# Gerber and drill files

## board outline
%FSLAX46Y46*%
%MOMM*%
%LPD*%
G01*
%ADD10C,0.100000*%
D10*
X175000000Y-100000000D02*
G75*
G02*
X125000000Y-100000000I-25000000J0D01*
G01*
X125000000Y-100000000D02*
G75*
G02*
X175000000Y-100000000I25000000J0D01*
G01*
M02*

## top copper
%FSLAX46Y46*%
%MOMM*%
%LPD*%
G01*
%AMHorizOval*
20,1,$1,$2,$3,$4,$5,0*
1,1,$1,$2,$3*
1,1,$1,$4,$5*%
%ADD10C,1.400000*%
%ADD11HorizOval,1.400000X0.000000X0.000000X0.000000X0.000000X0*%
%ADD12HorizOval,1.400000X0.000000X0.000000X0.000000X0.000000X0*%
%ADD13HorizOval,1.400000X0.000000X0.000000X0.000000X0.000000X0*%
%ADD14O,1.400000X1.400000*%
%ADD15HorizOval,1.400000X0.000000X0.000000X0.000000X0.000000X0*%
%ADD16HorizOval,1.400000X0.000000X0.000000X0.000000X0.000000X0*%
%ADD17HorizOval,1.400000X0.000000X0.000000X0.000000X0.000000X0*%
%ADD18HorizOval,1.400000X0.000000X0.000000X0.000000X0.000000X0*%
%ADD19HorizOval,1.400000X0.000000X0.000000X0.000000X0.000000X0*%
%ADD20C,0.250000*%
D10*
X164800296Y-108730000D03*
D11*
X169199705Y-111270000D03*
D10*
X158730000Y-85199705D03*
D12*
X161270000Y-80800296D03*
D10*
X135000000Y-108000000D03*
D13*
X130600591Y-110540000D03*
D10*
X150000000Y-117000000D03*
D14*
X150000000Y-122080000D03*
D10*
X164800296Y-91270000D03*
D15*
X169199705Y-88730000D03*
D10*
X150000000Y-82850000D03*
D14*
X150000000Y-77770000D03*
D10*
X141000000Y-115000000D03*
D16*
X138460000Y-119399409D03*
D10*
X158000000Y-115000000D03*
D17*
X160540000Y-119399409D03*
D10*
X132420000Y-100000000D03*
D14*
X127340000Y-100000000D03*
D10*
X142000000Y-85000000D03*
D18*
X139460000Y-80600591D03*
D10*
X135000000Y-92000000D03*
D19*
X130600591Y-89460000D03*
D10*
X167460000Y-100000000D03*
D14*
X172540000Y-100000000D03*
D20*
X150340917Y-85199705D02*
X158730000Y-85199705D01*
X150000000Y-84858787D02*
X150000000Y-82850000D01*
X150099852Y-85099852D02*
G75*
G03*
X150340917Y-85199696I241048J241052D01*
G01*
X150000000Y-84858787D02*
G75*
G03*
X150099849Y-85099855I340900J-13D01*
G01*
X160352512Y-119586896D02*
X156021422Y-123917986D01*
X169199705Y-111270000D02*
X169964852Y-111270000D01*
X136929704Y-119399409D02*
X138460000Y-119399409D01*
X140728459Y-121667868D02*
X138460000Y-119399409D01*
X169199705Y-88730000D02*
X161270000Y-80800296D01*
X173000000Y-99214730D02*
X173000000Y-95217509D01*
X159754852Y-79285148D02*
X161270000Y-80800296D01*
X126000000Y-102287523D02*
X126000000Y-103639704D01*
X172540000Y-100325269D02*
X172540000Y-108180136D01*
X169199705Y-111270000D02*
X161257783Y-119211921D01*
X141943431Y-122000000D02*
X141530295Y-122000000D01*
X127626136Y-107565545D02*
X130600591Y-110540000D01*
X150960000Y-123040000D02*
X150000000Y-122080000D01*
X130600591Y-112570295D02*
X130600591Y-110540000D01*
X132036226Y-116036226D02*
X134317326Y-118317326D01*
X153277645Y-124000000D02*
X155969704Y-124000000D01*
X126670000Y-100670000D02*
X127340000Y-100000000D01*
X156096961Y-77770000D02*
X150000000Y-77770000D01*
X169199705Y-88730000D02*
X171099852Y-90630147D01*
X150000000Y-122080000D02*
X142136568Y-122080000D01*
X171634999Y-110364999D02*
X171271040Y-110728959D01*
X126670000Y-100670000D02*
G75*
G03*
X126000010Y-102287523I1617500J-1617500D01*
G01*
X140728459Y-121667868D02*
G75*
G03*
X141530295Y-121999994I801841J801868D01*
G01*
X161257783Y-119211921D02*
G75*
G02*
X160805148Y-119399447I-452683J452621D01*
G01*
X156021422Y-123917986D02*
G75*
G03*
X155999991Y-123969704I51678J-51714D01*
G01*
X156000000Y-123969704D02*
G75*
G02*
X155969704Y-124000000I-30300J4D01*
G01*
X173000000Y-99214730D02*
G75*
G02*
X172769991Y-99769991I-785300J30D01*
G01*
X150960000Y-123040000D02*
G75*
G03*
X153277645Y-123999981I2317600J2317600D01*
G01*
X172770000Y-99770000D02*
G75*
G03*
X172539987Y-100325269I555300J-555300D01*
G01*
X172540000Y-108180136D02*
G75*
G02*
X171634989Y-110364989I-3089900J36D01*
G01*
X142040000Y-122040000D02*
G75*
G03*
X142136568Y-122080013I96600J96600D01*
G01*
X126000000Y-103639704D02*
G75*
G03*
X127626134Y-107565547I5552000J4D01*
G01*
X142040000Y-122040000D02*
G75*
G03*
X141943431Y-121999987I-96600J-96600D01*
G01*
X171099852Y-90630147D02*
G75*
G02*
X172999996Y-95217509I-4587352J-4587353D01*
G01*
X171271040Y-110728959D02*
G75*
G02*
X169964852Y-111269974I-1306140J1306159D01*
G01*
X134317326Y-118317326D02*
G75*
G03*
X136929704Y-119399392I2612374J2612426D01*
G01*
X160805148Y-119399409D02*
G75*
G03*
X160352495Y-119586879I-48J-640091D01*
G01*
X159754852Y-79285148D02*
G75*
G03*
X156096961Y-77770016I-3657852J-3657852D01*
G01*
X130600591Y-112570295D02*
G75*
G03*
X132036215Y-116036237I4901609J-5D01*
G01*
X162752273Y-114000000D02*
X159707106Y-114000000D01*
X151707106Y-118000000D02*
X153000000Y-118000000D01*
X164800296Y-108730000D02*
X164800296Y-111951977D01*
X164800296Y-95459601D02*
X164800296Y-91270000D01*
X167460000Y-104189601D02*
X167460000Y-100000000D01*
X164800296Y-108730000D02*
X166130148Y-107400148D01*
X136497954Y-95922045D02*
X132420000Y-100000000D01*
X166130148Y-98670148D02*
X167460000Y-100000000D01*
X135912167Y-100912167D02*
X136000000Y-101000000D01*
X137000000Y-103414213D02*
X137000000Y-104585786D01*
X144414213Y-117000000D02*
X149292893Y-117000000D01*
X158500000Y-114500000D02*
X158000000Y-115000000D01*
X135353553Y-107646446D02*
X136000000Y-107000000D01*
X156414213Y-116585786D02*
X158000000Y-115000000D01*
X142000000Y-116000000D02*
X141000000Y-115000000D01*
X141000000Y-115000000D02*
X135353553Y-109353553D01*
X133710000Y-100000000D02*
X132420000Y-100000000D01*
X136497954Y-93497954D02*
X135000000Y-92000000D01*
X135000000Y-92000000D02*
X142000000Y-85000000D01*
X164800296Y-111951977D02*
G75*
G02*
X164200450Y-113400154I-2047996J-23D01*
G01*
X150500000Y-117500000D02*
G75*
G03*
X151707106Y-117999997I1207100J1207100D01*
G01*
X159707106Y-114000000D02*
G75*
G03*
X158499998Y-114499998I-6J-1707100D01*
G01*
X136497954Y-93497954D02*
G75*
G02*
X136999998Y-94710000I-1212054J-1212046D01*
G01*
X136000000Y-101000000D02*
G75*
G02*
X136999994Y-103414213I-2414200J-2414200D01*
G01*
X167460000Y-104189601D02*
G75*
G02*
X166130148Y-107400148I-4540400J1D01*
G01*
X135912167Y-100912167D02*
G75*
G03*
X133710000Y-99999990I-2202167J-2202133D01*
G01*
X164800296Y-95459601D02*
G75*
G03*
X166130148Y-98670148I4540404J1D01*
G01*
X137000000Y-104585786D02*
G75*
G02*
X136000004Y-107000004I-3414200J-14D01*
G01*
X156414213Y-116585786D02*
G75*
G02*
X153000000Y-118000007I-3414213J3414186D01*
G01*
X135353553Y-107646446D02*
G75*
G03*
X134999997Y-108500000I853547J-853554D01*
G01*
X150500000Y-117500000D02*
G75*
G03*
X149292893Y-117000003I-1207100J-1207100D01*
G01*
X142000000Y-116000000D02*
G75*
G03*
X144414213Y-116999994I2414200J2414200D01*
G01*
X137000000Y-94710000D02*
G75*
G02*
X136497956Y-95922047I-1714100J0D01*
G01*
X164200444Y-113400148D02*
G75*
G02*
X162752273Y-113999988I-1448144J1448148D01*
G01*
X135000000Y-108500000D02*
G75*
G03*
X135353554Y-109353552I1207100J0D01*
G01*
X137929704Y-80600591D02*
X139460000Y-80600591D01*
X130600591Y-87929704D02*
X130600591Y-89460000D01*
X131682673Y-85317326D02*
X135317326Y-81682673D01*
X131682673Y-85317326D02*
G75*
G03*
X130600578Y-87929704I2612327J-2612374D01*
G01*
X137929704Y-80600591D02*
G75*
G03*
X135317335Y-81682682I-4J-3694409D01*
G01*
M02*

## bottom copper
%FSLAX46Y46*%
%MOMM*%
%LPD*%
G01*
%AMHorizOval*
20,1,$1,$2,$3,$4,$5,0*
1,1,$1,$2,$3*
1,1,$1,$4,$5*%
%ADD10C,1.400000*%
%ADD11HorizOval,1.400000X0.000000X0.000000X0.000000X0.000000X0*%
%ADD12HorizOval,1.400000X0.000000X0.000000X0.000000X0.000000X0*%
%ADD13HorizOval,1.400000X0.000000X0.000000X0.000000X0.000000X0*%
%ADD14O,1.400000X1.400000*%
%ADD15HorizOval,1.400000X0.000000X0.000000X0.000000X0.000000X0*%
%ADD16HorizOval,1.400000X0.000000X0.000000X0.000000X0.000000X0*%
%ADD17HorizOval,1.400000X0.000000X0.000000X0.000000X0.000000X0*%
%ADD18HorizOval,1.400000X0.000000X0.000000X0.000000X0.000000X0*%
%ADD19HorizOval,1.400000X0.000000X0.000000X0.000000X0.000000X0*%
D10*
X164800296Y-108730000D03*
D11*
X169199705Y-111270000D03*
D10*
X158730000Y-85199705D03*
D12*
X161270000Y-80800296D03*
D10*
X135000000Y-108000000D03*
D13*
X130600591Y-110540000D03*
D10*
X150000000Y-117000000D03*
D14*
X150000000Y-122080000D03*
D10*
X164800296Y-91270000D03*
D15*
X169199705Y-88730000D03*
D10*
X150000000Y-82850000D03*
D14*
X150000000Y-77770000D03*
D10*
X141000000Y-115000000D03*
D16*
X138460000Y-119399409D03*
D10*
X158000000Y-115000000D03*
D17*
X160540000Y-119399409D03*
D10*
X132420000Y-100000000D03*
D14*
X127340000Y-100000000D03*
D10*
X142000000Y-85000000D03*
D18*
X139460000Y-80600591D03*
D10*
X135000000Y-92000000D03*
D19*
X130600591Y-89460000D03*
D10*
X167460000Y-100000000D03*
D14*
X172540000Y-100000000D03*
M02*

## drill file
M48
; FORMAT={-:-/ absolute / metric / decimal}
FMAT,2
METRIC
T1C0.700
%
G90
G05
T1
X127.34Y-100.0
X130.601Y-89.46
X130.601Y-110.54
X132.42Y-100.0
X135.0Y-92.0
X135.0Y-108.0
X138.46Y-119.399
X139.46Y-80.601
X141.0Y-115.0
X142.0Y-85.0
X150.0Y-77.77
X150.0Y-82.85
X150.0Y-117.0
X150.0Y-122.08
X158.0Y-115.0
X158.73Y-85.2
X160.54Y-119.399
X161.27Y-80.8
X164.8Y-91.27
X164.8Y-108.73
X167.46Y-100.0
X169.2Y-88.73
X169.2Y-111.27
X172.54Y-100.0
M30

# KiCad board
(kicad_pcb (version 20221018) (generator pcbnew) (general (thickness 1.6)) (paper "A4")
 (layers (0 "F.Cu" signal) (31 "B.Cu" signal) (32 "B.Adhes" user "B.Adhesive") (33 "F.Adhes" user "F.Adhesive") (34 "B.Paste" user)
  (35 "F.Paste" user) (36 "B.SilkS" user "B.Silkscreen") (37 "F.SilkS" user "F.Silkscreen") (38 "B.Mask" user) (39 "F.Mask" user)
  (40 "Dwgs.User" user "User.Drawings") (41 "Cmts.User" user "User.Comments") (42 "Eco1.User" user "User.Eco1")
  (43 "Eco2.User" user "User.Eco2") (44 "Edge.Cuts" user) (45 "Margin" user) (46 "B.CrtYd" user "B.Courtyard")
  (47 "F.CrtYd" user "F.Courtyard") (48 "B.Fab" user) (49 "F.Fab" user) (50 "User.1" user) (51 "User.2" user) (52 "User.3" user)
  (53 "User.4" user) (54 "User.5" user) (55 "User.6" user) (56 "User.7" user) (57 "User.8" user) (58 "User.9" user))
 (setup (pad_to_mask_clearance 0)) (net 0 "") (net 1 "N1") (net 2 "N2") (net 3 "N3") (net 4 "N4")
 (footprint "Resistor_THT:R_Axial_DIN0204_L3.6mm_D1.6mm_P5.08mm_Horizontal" (layer "F.Cu") (at 164.800296 108.73 -30)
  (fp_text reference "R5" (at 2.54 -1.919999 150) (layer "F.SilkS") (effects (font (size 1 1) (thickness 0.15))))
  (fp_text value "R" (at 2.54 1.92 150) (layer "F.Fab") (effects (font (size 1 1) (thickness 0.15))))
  (pad "1" thru_hole circle (at 0 0 330) (size 1.4 1.4) (drill 0.7) (layers "*.Cu" "*.Mask") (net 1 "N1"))
  (pad "2" thru_hole oval (at 5.08 0 330) (size 1.4 1.4) (drill 0.7) (layers "*.Cu" "*.Mask") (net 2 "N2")))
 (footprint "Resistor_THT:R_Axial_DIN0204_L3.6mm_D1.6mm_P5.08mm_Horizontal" (layer "F.Cu") (at 158.73 85.199705 60)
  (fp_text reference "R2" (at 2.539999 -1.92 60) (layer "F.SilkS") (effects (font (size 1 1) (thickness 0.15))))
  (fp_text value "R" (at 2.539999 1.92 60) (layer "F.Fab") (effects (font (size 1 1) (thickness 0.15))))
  (pad "1" thru_hole circle (at 0 0 60) (size 1.4 1.4) (drill 0.7) (layers "*.Cu" "*.Mask") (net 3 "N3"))
  (pad "2" thru_hole oval (at 5.08 0 60) (size 1.4 1.4) (drill 0.7) (layers "*.Cu" "*.Mask") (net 2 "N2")))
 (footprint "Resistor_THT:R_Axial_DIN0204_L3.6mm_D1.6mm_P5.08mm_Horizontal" (layer "F.Cu") (at 135 108 -150)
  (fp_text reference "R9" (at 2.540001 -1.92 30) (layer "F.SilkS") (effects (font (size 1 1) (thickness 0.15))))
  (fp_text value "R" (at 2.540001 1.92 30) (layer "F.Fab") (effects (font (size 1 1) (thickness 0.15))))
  (pad "1" thru_hole circle (at 0 0 210) (size 1.4 1.4) (drill 0.7) (layers "*.Cu" "*.Mask") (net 1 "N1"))
  (pad "2" thru_hole oval (at 5.08 0 210) (size 1.4 1.4) (drill 0.7) (layers "*.Cu" "*.Mask") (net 2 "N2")))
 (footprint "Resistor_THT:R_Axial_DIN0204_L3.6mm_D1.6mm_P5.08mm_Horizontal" (layer "F.Cu") (at 150 117 -90)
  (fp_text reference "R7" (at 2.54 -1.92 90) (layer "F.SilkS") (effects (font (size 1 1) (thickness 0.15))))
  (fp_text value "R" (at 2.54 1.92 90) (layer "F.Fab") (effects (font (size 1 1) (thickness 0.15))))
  (pad "1" thru_hole circle (at 0 0 270) (size 1.4 1.4) (drill 0.7) (layers "*.Cu" "*.Mask") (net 1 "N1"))
  (pad "2" thru_hole oval (at 5.08 0 270) (size 1.4 1.4) (drill 0.7) (layers "*.Cu" "*.Mask") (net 2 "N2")))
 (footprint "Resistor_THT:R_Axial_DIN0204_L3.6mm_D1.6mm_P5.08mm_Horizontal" (layer "F.Cu") (at 164.800296 91.27 30)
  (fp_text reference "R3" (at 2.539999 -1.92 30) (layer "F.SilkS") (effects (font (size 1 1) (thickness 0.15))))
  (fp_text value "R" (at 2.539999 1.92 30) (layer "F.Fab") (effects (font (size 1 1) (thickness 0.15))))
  (pad "1" thru_hole circle (at 0 0 30) (size 1.4 1.4) (drill 0.7) (layers "*.Cu" "*.Mask") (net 1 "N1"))
  (pad "2" thru_hole oval (at 5.08 0 30) (size 1.4 1.4) (drill 0.7) (layers "*.Cu" "*.Mask") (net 2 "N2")))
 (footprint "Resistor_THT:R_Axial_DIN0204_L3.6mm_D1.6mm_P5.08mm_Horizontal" (layer "F.Cu") (at 150 82.85 90)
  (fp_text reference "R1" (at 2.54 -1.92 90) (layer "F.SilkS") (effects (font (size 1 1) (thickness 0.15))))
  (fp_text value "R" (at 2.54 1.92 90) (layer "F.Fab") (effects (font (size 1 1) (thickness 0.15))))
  (pad "1" thru_hole circle (at 0 0 90) (size 1.4 1.4) (drill 0.7) (layers "*.Cu" "*.Mask") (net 3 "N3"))
  (pad "2" thru_hole oval (at 5.08 0 90) (size 1.4 1.4) (drill 0.7) (layers "*.Cu" "*.Mask") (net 2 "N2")))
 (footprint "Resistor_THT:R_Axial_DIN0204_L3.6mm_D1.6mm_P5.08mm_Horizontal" (layer "F.Cu") (at 141 115 -120)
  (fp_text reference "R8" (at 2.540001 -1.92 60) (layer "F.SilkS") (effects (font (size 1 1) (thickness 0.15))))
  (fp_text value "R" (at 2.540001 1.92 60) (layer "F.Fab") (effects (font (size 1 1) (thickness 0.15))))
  (pad "1" thru_hole circle (at 0 0 240) (size 1.4 1.4) (drill 0.7) (layers "*.Cu" "*.Mask") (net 1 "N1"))
  (pad "2" thru_hole oval (at 5.08 0 240) (size 1.4 1.4) (drill 0.7) (layers "*.Cu" "*.Mask") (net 2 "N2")))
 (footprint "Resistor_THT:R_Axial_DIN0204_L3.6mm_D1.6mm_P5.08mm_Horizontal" (layer "F.Cu") (at 158 115 -60)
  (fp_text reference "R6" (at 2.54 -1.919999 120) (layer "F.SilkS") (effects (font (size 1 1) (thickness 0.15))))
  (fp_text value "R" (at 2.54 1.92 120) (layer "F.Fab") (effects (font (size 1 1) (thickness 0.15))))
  (pad "1" thru_hole circle (at 0 0 300) (size 1.4 1.4) (drill 0.7) (layers "*.Cu" "*.Mask") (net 1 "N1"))
  (pad "2" thru_hole oval (at 5.08 0 300) (size 1.4 1.4) (drill 0.7) (layers "*.Cu" "*.Mask") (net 2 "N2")))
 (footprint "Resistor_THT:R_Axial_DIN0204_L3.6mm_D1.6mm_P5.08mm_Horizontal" (layer "F.Cu") (at 132.42 100 180)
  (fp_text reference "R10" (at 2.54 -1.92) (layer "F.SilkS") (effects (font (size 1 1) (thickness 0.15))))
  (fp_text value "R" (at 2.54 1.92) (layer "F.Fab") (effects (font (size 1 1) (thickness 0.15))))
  (pad "1" thru_hole circle (at 0 0 180) (size 1.4 1.4) (drill 0.7) (layers "*.Cu" "*.Mask") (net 1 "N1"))
  (pad "2" thru_hole oval (at 5.08 0 180) (size 1.4 1.4) (drill 0.7) (layers "*.Cu" "*.Mask") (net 2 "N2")))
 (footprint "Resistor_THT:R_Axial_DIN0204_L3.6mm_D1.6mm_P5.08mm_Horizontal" (layer "F.Cu") (at 142 85 120)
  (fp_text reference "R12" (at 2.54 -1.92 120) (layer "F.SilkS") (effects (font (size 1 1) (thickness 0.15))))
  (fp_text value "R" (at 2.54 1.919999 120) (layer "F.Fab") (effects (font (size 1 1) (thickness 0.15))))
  (pad "1" thru_hole circle (at 0 0 120) (size 1.4 1.4) (drill 0.7) (layers "*.Cu" "*.Mask") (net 1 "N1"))
  (pad "2" thru_hole oval (at 5.08 0 120) (size 1.4 1.4) (drill 0.7) (layers "*.Cu" "*.Mask") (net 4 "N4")))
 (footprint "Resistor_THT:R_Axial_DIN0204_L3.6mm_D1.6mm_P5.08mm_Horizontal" (layer "F.Cu") (at 135 92 150)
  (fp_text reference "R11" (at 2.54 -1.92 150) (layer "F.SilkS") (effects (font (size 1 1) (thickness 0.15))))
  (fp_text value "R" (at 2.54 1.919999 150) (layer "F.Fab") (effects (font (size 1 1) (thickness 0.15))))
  (pad "1" thru_hole circle (at 0 0 150) (size 1.4 1.4) (drill 0.7) (layers "*.Cu" "*.Mask") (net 1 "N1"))
  (pad "2" thru_hole oval (at 5.08 0 150) (size 1.4 1.4) (drill 0.7) (layers "*.Cu" "*.Mask") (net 4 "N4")))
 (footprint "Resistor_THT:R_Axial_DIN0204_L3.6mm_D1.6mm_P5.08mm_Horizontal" (layer "F.Cu") (at 167.46 100)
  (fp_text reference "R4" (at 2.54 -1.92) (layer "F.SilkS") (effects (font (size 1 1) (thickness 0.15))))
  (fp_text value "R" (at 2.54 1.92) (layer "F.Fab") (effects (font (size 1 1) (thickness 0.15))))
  (pad "1" thru_hole circle (at 0 0) (size 1.4 1.4) (drill 0.7) (layers "*.Cu" "*.Mask") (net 1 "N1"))
  (pad "2" thru_hole oval (at 5.08 0) (size 1.4 1.4) (drill 0.7) (layers "*.Cu" "*.Mask") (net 2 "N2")))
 (gr_circle (center 150 100) (end 175 100) (stroke (width 0.1) (type default)) (fill none) (layer "Edge.Cuts"))
 (segment (start 150.340917 85.199705) (end 158.73 85.199705) (width 0.25) (layer "F.Cu") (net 3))
 (segment (start 150 84.858787) (end 150 82.85) (width 0.25) (layer "F.Cu") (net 3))
 (arc (start 150.099852 85.099852) (mid 150.210453 85.173754) (end 150.340917 85.199705) (width 0.25) (layer "F.Cu") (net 3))
 (arc (start 150 84.858787) (mid 150.02595 84.98925) (end 150.099852 85.099852) (width 0.25) (layer "F.Cu") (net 3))
 (segment (start 160.352512 119.586896) (end 156.021422 123.917986) (width 0.25) (layer "F.Cu") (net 2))
 (segment (start 169.199705 111.27) (end 169.964852 111.27) (width 0.25) (layer "F.Cu") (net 2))
 (segment (start 136.929704 119.399409) (end 138.46 119.399409) (width 0.25) (layer "F.Cu") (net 2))
 (segment (start 140.728459 121.667868) (end 138.46 119.399409) (width 0.25) (layer "F.Cu") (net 2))
 (segment (start 169.199705 88.73) (end 161.27 80.800296) (width 0.25) (layer "F.Cu") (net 2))
 (segment (start 173 99.21473) (end 173 95.217509) (width 0.25) (layer "F.Cu") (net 2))
 (segment (start 159.754852 79.285148) (end 161.27 80.800296) (width 0.25) (layer "F.Cu") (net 2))
 (segment (start 126 102.287523) (end 126 103.639704) (width 0.25) (layer "F.Cu") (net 2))
 (segment (start 172.54 100.325269) (end 172.54 108.180136) (width 0.25) (layer "F.Cu") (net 2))
 (segment (start 169.199705 111.27) (end 161.257783 119.211921) (width 0.25) (layer "F.Cu") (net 2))
 (segment (start 141.943431 122) (end 141.530295 122) (width 0.25) (layer "F.Cu") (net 2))
 (segment (start 127.626136 107.565545) (end 130.600591 110.54) (width 0.25) (layer "F.Cu") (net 2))
 (segment (start 150.96 123.04) (end 150 122.08) (width 0.25) (layer "F.Cu") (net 2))
 (segment (start 130.600591 112.570295) (end 130.600591 110.54) (width 0.25) (layer "F.Cu") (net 2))
 (segment (start 132.036226 116.036226) (end 134.317326 118.317326) (width 0.25) (layer "F.Cu") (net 2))
 (segment (start 153.277645 124) (end 155.969704 124) (width 0.25) (layer "F.Cu") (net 2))
 (segment (start 126.67 100.67) (end 127.34 100) (width 0.25) (layer "F.Cu") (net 2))
 (segment (start 156.096961 77.77) (end 150 77.77) (width 0.25) (layer "F.Cu") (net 2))
 (segment (start 169.199705 88.73) (end 171.099852 90.630147) (width 0.25) (layer "F.Cu") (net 2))
 (segment (start 150 122.08) (end 142.136568 122.08) (width 0.25) (layer "F.Cu") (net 2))
 (segment (start 171.634999 110.364999) (end 171.27104 110.728959) (width 0.25) (layer "F.Cu") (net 2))
 (arc (start 126.67 100.67) (mid 126.174127 101.412125) (end 126 102.287523) (width 0.25) (layer "F.Cu") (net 2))
 (arc (start 140.728459 121.667868) (mid 141.096344 121.913681) (end 141.530295 122) (width 0.25) (layer "F.Cu") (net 2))
 (arc (start 161.257783 119.211921) (mid 161.050112 119.350682) (end 160.805148 119.399409) (width 0.25) (layer "F.Cu") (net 2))
 (arc (start 156.021422 123.917986) (mid 156.005567 123.941714) (end 156 123.969704) (width 0.25) (layer "F.Cu") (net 2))
 (arc (start 156 123.969704) (mid 155.991126 123.991126) (end 155.969704 124) (width 0.25) (layer "F.Cu") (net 2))
 (arc (start 173 99.21473) (mid 172.940224 99.51524) (end 172.77 99.77) (width 0.25) (layer "F.Cu") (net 2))
 (arc (start 150.96 123.04) (mid 152.023344 123.750504) (end 153.277645 124) (width 0.25) (layer "F.Cu") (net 2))
 (arc (start 172.77 99.77) (mid 172.599775 100.024759) (end 172.54 100.325269) (width 0.25) (layer "F.Cu") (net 2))
 (arc (start 172.54 108.180136) (mid 172.304797 109.362575) (end 171.634999 110.364999) (width 0.25) (layer "F.Cu") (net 2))
 (arc (start 142.04 122.04) (mid 142.084305 122.069604) (end 142.136568 122.08) (width 0.25) (layer "F.Cu") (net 2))
 (arc (start 126 103.639704) (mid 126.422618 105.764354) (end 127.626136 107.565545) (width 0.25) (layer "F.Cu") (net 2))
 (arc (start 142.04 122.04) (mid 141.995693 122.010395) (end 141.943431 122) (width 0.25) (layer "F.Cu") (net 2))
 (arc (start 171.099852 90.630147) (mid 172.506167 92.734846) (end 173 95.217509) (width 0.25) (layer "F.Cu") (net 2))
 (arc (start 171.27104 110.728959) (mid 170.671756 111.129388) (end 169.964852 111.27) (width 0.25) (layer "F.Cu") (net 2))
 (arc (start 134.317326 118.317326) (mid 135.515895 119.118184) (end 136.929704 119.399409) (width 0.25) (layer "F.Cu") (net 2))
 (arc (start 160.805148 119.399409) (mid 160.560183 119.448135) (end 160.352512 119.586896) (width 0.25) (layer "F.Cu") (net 2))
 (arc (start 159.754852 79.285148) (mid 158.076597 78.163774) (end 156.096961 77.77) (width 0.25) (layer "F.Cu") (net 2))
 (arc (start 130.600591 112.570295) (mid 130.9737 114.446043) (end 132.036226 116.036226) (width 0.25) (layer "F.Cu") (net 2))
 (segment (start 162.752273 114) (end 159.707106 114) (width 0.25) (layer "F.Cu") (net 1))
 (segment (start 151.707106 118) (end 153 118) (width 0.25) (layer "F.Cu") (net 1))
 (segment (start 164.800296 108.73) (end 164.800296 111.951977) (width 0.25) (layer "F.Cu") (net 1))
 (segment (start 164.800296 95.459601) (end 164.800296 91.27) (width 0.25) (layer "F.Cu") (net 1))
 (segment (start 167.46 104.189601) (end 167.46 100) (width 0.25) (layer "F.Cu") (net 1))
 (segment (start 164.800296 108.73) (end 166.130148 107.400148) (width 0.25) (layer "F.Cu") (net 1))
 (segment (start 136.497954 95.922045) (end 132.42 100) (width 0.25) (layer "F.Cu") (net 1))
 (segment (start 166.130148 98.670148) (end 167.46 100) (width 0.25) (layer "F.Cu") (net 1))
 (segment (start 135.912167 100.912167) (end 136 101) (width 0.25) (layer "F.Cu") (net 1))
 (segment (start 137 103.414213) (end 137 104.585786) (width 0.25) (layer "F.Cu") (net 1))
 (segment (start 144.414213 117) (end 149.292893 117) (width 0.25) (layer "F.Cu") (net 1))
 (segment (start 158.5 114.5) (end 158 115) (width 0.25) (layer "F.Cu") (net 1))
 (segment (start 135.353553 107.646446) (end 136 107) (width 0.25) (layer "F.Cu") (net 1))
 (segment (start 156.414213 116.585786) (end 158 115) (width 0.25) (layer "F.Cu") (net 1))
 (segment (start 142 116) (end 141 115) (width 0.25) (layer "F.Cu") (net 1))
 (segment (start 141 115) (end 135.353553 109.353553) (width 0.25) (layer "F.Cu") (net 1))
 (segment (start 133.71 100) (end 132.42 100) (width 0.25) (layer "F.Cu") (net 1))
 (segment (start 136.497954 93.497954) (end 135 92) (width 0.25) (layer "F.Cu") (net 1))
 (segment (start 135 92) (end 142 85) (width 0.25) (layer "F.Cu") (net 1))
 (arc (start 164.800296 111.951977) (mid 164.644399 112.735721) (end 164.200444 113.400148) (width 0.25) (layer "F.Cu") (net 1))
 (arc (start 150.5 117.5) (mid 151.053825 117.870054) (end 151.707106 118) (width 0.25) (layer "F.Cu") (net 1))
 (arc (start 159.707106 114) (mid 159.053825 114.129945) (end 158.5 114.5) (width 0.25) (layer "F.Cu") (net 1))
 (arc (start 136.497954 93.497954) (mid 136.869522 94.054045) (end 137 94.71) (width 0.25) (layer "F.Cu") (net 1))
 (arc (start 136 101) (mid 136.740108 102.10765) (end 137 103.414213) (width 0.25) (layer "F.Cu") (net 1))
 (arc (start 167.46 104.189601) (mid 167.114382 105.927136) (end 166.130148 107.400148) (width 0.25) (layer "F.Cu") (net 1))
 (arc (start 135.912167 100.912167) (mid 134.901804 100.237064) (end 133.71 100) (width 0.25) (layer "F.Cu") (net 1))
 (arc (start 164.800296 95.459601) (mid 165.145913 97.197136) (end 166.130148 98.670148) (width 0.25) (layer "F.Cu") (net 1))
 (arc (start 137 104.585786) (mid 136.740108 105.892349) (end 136 107) (width 0.25) (layer "F.Cu") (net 1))
 (arc (start 156.414213 116.585786) (mid 154.847758 117.632457) (end 153 118) (width 0.25) (layer "F.Cu") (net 1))
 (arc (start 135.353553 107.646446) (mid 135.091885 108.03806) (end 135 108.5) (width 0.25) (layer "F.Cu") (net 1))
 (arc (start 150.5 117.5) (mid 149.946174 117.129945) (end 149.292893 117) (width 0.25) (layer "F.Cu") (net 1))
 (arc (start 142 116) (mid 143.10765 116.740108) (end 144.414213 117) (width 0.25) (layer "F.Cu") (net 1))
 (arc (start 137 94.71) (mid 136.869522 95.365954) (end 136.497954 95.922045) (width 0.25) (layer "F.Cu") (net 1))
 (arc (start 164.200444 113.400148) (mid 163.536017 113.844103) (end 162.752273 114) (width 0.25) (layer "F.Cu") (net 1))
 (arc (start 135 108.5) (mid 135.091885 108.961939) (end 135.353553 109.353553) (width 0.25) (layer "F.Cu") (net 1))
 (segment (start 137.929704 80.600591) (end 139.46 80.600591) (width 0.25) (layer "F.Cu") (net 4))
 (segment (start 130.600591 87.929704) (end 130.600591 89.46) (width 0.25) (layer "F.Cu") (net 4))
 (segment (start 131.682673 85.317326) (end 135.317326 81.682673) (width 0.25) (layer "F.Cu") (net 4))
 (arc (start 131.682673 85.317326) (mid 130.881814 86.515895) (end 130.600591 87.929704) (width 0.25) (layer "F.Cu") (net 4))
 (arc (start 137.929704 80.600591) (mid 136.515895 80.881814) (end 135.317326 81.682673) (width 0.25) (layer "F.Cu") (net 4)))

